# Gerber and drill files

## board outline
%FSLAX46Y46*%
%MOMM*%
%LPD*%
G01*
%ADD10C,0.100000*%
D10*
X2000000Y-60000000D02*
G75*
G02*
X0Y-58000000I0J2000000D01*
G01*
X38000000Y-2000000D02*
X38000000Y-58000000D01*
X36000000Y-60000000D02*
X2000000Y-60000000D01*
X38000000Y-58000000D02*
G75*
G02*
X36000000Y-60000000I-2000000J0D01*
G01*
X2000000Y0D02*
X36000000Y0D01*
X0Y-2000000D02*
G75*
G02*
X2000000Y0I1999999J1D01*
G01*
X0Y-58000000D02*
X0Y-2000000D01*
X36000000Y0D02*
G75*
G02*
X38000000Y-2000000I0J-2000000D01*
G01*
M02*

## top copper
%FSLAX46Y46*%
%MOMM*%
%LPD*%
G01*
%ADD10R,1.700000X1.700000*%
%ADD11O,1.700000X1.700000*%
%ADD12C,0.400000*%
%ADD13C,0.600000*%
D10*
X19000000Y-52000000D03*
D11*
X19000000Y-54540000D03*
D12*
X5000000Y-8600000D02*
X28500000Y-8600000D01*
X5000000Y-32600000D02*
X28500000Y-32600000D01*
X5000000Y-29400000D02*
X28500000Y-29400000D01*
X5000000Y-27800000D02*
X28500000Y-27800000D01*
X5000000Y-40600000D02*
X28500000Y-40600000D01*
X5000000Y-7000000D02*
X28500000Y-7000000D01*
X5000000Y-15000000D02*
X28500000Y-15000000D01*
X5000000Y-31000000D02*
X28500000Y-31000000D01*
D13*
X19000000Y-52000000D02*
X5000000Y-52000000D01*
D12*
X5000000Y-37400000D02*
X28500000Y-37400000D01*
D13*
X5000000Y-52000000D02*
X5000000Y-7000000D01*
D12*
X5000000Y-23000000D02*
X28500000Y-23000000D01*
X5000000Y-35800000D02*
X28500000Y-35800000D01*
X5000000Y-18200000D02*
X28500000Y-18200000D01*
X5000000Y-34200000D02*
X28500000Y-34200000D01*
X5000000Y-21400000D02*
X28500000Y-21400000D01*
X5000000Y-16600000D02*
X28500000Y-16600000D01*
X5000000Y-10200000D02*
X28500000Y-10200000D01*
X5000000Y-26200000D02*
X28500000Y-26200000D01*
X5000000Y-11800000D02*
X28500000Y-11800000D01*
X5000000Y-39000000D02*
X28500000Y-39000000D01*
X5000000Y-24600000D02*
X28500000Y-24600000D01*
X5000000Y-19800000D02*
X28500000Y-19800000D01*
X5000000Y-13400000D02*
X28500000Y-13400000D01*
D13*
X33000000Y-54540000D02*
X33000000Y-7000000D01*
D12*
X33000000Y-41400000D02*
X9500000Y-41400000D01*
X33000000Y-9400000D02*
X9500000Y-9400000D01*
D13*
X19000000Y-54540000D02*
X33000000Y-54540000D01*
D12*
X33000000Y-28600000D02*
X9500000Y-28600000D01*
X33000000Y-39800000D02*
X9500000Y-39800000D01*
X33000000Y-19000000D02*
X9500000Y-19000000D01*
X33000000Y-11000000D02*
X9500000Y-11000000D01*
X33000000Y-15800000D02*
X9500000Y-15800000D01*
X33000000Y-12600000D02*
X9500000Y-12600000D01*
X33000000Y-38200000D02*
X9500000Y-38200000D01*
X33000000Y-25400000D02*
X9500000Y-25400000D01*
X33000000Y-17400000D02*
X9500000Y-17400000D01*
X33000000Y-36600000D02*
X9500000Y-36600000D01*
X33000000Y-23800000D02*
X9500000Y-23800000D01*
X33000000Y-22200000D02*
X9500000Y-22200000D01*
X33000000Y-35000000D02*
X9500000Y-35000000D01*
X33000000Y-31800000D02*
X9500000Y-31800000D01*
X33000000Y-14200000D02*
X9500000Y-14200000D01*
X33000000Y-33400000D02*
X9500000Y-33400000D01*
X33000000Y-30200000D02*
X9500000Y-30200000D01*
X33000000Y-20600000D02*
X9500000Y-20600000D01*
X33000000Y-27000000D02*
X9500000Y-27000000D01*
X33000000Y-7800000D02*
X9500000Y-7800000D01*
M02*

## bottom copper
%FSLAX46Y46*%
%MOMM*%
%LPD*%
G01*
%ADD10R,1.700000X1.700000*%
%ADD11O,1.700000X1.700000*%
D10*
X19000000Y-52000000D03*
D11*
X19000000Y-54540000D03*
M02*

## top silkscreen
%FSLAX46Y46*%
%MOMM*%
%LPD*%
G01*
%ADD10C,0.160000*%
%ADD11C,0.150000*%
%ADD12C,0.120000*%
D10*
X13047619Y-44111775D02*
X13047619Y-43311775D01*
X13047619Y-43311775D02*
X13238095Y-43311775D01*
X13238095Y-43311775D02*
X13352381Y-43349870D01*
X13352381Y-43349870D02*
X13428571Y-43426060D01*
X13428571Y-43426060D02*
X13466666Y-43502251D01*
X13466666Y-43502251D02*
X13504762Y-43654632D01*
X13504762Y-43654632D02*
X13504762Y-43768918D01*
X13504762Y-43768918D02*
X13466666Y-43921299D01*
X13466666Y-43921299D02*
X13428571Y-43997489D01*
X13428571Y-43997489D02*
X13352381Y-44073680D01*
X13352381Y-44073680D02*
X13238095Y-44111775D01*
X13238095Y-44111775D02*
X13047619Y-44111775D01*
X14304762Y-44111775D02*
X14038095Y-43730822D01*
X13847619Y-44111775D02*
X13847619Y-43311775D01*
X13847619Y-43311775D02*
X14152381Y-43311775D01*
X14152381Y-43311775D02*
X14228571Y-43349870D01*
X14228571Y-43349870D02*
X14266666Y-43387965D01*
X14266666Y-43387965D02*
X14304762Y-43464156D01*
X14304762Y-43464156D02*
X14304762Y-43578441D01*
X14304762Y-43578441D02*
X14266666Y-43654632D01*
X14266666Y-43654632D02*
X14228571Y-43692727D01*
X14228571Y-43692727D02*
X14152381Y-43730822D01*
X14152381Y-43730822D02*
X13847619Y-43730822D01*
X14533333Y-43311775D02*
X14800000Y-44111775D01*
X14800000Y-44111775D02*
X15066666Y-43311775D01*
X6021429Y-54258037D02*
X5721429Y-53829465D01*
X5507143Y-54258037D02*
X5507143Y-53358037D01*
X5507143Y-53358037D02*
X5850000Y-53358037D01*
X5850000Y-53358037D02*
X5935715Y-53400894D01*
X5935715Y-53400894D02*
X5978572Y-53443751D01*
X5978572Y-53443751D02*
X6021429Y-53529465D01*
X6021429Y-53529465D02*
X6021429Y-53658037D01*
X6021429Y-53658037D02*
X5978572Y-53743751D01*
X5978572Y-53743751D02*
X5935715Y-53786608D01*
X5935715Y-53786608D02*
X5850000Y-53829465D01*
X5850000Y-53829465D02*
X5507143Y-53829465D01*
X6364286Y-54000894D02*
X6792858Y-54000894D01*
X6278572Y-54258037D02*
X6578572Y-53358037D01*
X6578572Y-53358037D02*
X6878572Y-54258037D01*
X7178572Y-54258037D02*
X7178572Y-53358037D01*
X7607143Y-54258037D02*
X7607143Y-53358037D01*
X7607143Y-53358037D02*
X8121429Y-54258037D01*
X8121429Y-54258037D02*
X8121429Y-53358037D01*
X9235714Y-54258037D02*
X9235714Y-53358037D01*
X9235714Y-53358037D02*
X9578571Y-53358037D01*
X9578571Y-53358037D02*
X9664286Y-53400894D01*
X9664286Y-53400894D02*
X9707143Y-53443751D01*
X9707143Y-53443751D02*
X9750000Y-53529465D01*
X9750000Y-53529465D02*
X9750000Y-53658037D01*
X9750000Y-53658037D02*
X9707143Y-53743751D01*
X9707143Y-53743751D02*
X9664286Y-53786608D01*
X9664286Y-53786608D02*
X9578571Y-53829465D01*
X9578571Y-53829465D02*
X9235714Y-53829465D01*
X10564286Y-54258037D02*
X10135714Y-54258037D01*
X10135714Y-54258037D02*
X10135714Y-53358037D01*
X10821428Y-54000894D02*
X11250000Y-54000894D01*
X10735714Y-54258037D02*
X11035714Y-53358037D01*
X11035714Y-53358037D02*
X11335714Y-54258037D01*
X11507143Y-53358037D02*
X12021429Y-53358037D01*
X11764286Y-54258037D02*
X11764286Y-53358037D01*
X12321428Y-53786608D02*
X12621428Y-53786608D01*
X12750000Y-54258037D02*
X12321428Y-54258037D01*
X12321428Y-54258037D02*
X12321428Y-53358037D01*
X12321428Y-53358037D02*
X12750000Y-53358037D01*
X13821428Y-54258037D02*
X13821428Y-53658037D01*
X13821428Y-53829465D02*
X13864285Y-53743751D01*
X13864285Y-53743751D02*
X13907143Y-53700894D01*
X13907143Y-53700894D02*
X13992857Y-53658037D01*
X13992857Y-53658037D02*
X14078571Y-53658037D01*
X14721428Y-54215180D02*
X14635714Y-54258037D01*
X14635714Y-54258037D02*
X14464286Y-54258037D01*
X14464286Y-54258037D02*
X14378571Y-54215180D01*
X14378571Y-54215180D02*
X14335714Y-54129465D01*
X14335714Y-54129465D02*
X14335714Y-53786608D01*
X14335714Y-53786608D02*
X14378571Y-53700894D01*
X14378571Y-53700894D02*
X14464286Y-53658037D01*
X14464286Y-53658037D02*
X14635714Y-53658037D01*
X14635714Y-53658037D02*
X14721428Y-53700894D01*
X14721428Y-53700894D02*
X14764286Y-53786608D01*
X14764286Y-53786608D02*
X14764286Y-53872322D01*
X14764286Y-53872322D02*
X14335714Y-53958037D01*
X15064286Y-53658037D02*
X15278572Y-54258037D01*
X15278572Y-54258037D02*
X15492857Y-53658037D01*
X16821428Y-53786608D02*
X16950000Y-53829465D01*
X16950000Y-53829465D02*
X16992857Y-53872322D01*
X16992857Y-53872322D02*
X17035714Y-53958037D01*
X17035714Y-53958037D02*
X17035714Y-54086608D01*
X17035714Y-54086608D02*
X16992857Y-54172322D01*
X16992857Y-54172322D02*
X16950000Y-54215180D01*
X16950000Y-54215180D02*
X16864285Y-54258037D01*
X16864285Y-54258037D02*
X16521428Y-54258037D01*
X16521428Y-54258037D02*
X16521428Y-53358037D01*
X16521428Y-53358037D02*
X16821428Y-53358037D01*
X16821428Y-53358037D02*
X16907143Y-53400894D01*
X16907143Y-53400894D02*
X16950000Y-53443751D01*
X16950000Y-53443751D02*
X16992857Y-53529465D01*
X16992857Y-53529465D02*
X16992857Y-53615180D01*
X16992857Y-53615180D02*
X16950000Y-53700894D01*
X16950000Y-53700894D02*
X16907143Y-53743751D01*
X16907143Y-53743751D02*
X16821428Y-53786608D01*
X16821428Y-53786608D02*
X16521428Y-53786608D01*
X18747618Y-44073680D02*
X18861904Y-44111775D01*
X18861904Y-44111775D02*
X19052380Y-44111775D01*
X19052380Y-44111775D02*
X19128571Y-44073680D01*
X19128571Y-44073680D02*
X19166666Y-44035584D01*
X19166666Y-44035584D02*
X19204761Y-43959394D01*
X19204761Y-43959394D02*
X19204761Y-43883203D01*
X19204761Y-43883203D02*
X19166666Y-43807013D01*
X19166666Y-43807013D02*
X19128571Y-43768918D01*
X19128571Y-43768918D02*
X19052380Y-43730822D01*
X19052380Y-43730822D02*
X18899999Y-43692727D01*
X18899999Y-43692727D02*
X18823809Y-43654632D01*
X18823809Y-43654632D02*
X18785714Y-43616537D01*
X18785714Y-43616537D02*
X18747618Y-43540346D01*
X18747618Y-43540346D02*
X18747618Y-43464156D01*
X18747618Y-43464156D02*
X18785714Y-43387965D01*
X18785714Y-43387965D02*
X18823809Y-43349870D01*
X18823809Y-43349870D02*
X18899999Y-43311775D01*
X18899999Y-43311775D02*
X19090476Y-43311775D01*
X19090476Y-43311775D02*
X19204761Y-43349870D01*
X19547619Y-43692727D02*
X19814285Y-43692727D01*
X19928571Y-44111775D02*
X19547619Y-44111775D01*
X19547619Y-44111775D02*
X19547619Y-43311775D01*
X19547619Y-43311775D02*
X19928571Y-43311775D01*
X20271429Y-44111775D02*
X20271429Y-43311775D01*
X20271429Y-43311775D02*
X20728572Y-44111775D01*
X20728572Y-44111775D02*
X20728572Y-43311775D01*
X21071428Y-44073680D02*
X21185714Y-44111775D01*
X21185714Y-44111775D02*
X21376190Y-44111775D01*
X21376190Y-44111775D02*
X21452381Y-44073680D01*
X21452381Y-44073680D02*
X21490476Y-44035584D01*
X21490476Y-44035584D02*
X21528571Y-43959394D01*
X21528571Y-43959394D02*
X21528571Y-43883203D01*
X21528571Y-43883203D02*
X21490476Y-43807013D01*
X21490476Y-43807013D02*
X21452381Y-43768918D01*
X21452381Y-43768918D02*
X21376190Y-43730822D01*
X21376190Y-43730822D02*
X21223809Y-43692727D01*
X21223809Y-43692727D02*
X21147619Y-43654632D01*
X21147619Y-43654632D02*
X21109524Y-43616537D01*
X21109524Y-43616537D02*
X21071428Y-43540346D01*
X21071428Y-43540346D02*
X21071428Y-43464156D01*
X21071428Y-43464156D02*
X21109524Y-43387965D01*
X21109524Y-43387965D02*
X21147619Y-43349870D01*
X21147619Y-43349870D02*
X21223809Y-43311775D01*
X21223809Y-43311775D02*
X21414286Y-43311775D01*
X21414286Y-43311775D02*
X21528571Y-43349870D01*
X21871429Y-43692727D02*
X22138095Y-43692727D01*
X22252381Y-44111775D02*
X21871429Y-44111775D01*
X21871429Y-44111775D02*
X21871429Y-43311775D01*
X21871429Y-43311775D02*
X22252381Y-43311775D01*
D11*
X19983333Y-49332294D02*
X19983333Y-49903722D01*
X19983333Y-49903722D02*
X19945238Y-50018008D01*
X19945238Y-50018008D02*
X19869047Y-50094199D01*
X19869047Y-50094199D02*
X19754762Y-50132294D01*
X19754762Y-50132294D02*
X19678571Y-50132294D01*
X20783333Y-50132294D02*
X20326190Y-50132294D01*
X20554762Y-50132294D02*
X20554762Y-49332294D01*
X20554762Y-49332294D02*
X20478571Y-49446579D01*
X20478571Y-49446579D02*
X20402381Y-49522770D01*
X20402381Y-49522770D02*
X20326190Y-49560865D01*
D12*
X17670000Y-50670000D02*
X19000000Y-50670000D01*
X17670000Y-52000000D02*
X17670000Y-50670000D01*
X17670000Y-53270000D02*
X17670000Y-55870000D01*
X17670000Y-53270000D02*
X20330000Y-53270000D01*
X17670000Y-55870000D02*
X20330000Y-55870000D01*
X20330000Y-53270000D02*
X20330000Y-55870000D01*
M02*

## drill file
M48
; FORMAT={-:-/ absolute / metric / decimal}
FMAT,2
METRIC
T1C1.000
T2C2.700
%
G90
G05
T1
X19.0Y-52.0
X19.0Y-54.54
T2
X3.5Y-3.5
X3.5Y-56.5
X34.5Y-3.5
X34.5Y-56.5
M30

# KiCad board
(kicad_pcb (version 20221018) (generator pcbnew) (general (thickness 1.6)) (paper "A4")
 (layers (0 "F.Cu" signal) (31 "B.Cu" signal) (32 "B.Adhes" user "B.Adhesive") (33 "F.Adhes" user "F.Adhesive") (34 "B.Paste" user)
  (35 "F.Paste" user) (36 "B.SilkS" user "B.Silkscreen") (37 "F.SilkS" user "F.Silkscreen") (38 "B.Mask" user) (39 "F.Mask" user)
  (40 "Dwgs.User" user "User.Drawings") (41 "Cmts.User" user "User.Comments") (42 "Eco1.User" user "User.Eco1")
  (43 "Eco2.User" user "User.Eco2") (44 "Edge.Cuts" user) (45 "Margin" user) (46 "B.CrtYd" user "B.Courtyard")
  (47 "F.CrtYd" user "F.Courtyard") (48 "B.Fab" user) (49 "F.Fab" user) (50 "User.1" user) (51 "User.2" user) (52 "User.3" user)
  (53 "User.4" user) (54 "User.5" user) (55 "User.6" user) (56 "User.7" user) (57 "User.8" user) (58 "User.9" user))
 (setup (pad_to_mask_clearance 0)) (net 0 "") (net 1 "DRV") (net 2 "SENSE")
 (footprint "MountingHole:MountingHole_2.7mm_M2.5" (layer "F.Cu") (at 3.5 56.5)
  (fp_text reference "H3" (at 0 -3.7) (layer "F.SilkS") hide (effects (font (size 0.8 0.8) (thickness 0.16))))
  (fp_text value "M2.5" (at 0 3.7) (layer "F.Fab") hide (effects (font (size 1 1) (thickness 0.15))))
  (pad "" np_thru_hole circle (at 0 0) (size 2.7 2.7) (drill 2.7) (layers "*.Cu" "*.Mask")))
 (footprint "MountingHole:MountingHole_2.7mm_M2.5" (layer "F.Cu") (at 3.5 3.5)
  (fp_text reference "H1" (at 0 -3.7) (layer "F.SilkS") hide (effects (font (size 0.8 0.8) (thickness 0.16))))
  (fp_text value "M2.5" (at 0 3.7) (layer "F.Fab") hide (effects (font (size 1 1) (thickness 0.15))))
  (pad "" np_thru_hole circle (at 0 0) (size 2.7 2.7) (drill 2.7) (layers "*.Cu" "*.Mask")))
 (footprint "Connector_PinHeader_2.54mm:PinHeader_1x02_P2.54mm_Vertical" (layer "F.Cu") (at 19 52)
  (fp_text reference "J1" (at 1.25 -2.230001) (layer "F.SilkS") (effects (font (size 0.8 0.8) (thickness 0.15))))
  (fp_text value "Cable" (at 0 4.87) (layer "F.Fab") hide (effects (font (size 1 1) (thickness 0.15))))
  (fp_line (start -1.33 -1.33) (end 0 -1.33) (stroke (width 0.12) (type solid)) (layer "F.SilkS"))
  (fp_line (start -1.33 0) (end -1.33 -1.33) (stroke (width 0.12) (type solid)) (layer "F.SilkS"))
  (fp_line (start -1.33 1.27) (end -1.33 3.87) (stroke (width 0.12) (type solid)) (layer "F.SilkS"))
  (fp_line (start -1.33 1.27) (end 1.33 1.27) (stroke (width 0.12) (type solid)) (layer "F.SilkS"))
  (fp_line (start -1.33 3.87) (end 1.33 3.87) (stroke (width 0.12) (type solid)) (layer "F.SilkS"))
  (fp_line (start 1.33 1.27) (end 1.33 3.87) (stroke (width 0.12) (type solid)) (layer "F.SilkS"))
  (pad "1" thru_hole rect (at 0 0) (size 1.7 1.7) (drill 1) (layers "*.Cu" "*.Mask") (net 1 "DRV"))
  (pad "2" thru_hole oval (at 0 2.54) (size 1.7 1.7) (drill 1) (layers "*.Cu" "*.Mask") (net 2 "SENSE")))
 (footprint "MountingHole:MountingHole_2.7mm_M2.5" (layer "F.Cu") (at 34.5 3.5)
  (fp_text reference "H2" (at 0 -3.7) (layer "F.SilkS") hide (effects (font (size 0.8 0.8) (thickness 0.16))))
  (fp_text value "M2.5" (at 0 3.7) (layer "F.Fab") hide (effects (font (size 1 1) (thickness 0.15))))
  (pad "" np_thru_hole circle (at 0 0) (size 2.7 2.7) (drill 2.7) (layers "*.Cu" "*.Mask")))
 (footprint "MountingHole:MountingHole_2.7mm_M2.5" (layer "F.Cu") (at 34.5 56.5)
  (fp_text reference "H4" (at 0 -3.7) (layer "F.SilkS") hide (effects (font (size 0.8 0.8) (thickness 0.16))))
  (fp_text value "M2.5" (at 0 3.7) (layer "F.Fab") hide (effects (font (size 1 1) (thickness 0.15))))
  (pad "" np_thru_hole circle (at 0 0) (size 2.7 2.7) (drill 2.7) (layers "*.Cu" "*.Mask")))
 (gr_arc (start 2 60) (mid 0.585786 59.414213) (end 0 58) (stroke (width 0.1) (type default)) (layer "Edge.Cuts"))
 (gr_line (start 38 2) (end 38 58) (stroke (width 0.1) (type default)) (layer "Edge.Cuts"))
 (gr_line (start 36 60) (end 2 60) (stroke (width 0.1) (type default)) (layer "Edge.Cuts"))
 (gr_arc (start 38 58) (mid 37.414213 59.414213) (end 36 60) (stroke (width 0.1) (type default)) (layer "Edge.Cuts"))
 (gr_line (start 2 0) (end 36 0) (stroke (width 0.1) (type default)) (layer "Edge.Cuts"))
 (gr_arc (start 0 2) (mid 0.585786 0.585786) (end 2 0) (stroke (width 0.1) (type default)) (layer "Edge.Cuts"))
 (gr_line (start 0 58) (end 0 2) (stroke (width 0.1) (type default)) (layer "Edge.Cuts"))
 (gr_arc (start 36 0) (mid 37.414213 0.585786) (end 38 2) (stroke (width 0.1) (type default)) (layer "Edge.Cuts"))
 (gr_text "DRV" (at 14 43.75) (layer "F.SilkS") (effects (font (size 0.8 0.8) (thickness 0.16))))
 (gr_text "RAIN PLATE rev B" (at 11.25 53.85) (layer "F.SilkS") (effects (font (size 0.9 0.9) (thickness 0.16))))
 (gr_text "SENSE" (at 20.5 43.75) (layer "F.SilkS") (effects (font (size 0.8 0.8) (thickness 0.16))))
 (segment (start 5 8.6) (end 28.5 8.6) (width 0.4) (layer "F.Cu") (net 1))
 (segment (start 5 32.6) (end 28.5 32.6) (width 0.4) (layer "F.Cu") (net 1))
 (segment (start 5 29.4) (end 28.5 29.4) (width 0.4) (layer "F.Cu") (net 1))
 (segment (start 5 27.8) (end 28.5 27.8) (width 0.4) (layer "F.Cu") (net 1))
 (segment (start 5 40.6) (end 28.5 40.6) (width 0.4) (layer "F.Cu") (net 1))
 (segment (start 5 7) (end 28.5 7) (width 0.4) (layer "F.Cu") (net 1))
 (segment (start 5 15) (end 28.5 15) (width 0.4) (layer "F.Cu") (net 1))
 (segment (start 5 31) (end 28.5 31) (width 0.4) (layer "F.Cu") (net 1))
 (segment (start 19 52) (end 5 52) (width 0.6) (layer "F.Cu") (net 1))
 (segment (start 5 37.4) (end 28.5 37.4) (width 0.4) (layer "F.Cu") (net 1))
 (segment (start 5 52) (end 5 7) (width 0.6) (layer "F.Cu") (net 1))
 (segment (start 5 23) (end 28.5 23) (width 0.4) (layer "F.Cu") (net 1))
 (segment (start 5 35.8) (end 28.5 35.8) (width 0.4) (layer "F.Cu") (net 1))
 (segment (start 5 18.2) (end 28.5 18.2) (width 0.4) (layer "F.Cu") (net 1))
 (segment (start 5 34.2) (end 28.5 34.2) (width 0.4) (layer "F.Cu") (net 1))
 (segment (start 5 21.4) (end 28.5 21.4) (width 0.4) (layer "F.Cu") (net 1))
 (segment (start 5 16.6) (end 28.5 16.6) (width 0.4) (layer "F.Cu") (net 1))
 (segment (start 5 10.2) (end 28.5 10.2) (width 0.4) (layer "F.Cu") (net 1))
 (segment (start 5 26.2) (end 28.5 26.2) (width 0.4) (layer "F.Cu") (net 1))
 (segment (start 5 11.8) (end 28.5 11.8) (width 0.4) (layer "F.Cu") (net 1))
 (segment (start 5 39) (end 28.5 39) (width 0.4) (layer "F.Cu") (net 1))
 (segment (start 5 24.6) (end 28.5 24.6) (width 0.4) (layer "F.Cu") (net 1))
 (segment (start 5 19.8) (end 28.5 19.8) (width 0.4) (layer "F.Cu") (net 1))
 (segment (start 5 13.4) (end 28.5 13.4) (width 0.4) (layer "F.Cu") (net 1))
 (segment (start 33 54.54) (end 33 7) (width 0.6) (layer "F.Cu") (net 2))
 (segment (start 33 41.4) (end 9.5 41.4) (width 0.4) (layer "F.Cu") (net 2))
 (segment (start 33 9.4) (end 9.5 9.4) (width 0.4) (layer "F.Cu") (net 2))
 (segment (start 19 54.54) (end 33 54.54) (width 0.6) (layer "F.Cu") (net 2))
 (segment (start 33 28.6) (end 9.5 28.6) (width 0.4) (layer "F.Cu") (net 2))
 (segment (start 33 39.8) (end 9.5 39.8) (width 0.4) (layer "F.Cu") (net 2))
 (segment (start 33 19) (end 9.5 19) (width 0.4) (layer "F.Cu") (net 2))
 (segment (start 33 11) (end 9.5 11) (width 0.4) (layer "F.Cu") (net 2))
 (segment (start 33 15.8) (end 9.5 15.8) (width 0.4) (layer "F.Cu") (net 2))
 (segment (start 33 12.6) (end 9.5 12.6) (width 0.4) (layer "F.Cu") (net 2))
 (segment (start 33 38.2) (end 9.5 38.2) (width 0.4) (layer "F.Cu") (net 2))
 (segment (start 33 25.4) (end 9.5 25.4) (width 0.4) (layer "F.Cu") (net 2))
 (segment (start 33 17.4) (end 9.5 17.4) (width 0.4) (layer "F.Cu") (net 2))
 (segment (start 33 36.6) (end 9.5 36.6) (width 0.4) (layer "F.Cu") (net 2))
 (segment (start 33 23.8) (end 9.5 23.8) (width 0.4) (layer "F.Cu") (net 2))
 (segment (start 33 22.2) (end 9.5 22.2) (width 0.4) (layer "F.Cu") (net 2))
 (segment (start 33 35) (end 9.5 35) (width 0.4) (layer "F.Cu") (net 2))
 (segment (start 33 31.8) (end 9.5 31.8) (width 0.4) (layer "F.Cu") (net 2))
 (segment (start 33 14.2) (end 9.5 14.2) (width 0.4) (layer "F.Cu") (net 2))
 (segment (start 33 33.4) (end 9.5 33.4) (width 0.4) (layer "F.Cu") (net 2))
 (segment (start 33 30.2) (end 9.5 30.2) (width 0.4) (layer "F.Cu") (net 2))
 (segment (start 33 20.6) (end 9.5 20.6) (width 0.4) (layer "F.Cu") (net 2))
 (segment (start 33 27) (end 9.5 27) (width 0.4) (layer "F.Cu") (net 2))
 (segment (start 33 7.8) (end 9.5 7.8) (width 0.4) (layer "F.Cu") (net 2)))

